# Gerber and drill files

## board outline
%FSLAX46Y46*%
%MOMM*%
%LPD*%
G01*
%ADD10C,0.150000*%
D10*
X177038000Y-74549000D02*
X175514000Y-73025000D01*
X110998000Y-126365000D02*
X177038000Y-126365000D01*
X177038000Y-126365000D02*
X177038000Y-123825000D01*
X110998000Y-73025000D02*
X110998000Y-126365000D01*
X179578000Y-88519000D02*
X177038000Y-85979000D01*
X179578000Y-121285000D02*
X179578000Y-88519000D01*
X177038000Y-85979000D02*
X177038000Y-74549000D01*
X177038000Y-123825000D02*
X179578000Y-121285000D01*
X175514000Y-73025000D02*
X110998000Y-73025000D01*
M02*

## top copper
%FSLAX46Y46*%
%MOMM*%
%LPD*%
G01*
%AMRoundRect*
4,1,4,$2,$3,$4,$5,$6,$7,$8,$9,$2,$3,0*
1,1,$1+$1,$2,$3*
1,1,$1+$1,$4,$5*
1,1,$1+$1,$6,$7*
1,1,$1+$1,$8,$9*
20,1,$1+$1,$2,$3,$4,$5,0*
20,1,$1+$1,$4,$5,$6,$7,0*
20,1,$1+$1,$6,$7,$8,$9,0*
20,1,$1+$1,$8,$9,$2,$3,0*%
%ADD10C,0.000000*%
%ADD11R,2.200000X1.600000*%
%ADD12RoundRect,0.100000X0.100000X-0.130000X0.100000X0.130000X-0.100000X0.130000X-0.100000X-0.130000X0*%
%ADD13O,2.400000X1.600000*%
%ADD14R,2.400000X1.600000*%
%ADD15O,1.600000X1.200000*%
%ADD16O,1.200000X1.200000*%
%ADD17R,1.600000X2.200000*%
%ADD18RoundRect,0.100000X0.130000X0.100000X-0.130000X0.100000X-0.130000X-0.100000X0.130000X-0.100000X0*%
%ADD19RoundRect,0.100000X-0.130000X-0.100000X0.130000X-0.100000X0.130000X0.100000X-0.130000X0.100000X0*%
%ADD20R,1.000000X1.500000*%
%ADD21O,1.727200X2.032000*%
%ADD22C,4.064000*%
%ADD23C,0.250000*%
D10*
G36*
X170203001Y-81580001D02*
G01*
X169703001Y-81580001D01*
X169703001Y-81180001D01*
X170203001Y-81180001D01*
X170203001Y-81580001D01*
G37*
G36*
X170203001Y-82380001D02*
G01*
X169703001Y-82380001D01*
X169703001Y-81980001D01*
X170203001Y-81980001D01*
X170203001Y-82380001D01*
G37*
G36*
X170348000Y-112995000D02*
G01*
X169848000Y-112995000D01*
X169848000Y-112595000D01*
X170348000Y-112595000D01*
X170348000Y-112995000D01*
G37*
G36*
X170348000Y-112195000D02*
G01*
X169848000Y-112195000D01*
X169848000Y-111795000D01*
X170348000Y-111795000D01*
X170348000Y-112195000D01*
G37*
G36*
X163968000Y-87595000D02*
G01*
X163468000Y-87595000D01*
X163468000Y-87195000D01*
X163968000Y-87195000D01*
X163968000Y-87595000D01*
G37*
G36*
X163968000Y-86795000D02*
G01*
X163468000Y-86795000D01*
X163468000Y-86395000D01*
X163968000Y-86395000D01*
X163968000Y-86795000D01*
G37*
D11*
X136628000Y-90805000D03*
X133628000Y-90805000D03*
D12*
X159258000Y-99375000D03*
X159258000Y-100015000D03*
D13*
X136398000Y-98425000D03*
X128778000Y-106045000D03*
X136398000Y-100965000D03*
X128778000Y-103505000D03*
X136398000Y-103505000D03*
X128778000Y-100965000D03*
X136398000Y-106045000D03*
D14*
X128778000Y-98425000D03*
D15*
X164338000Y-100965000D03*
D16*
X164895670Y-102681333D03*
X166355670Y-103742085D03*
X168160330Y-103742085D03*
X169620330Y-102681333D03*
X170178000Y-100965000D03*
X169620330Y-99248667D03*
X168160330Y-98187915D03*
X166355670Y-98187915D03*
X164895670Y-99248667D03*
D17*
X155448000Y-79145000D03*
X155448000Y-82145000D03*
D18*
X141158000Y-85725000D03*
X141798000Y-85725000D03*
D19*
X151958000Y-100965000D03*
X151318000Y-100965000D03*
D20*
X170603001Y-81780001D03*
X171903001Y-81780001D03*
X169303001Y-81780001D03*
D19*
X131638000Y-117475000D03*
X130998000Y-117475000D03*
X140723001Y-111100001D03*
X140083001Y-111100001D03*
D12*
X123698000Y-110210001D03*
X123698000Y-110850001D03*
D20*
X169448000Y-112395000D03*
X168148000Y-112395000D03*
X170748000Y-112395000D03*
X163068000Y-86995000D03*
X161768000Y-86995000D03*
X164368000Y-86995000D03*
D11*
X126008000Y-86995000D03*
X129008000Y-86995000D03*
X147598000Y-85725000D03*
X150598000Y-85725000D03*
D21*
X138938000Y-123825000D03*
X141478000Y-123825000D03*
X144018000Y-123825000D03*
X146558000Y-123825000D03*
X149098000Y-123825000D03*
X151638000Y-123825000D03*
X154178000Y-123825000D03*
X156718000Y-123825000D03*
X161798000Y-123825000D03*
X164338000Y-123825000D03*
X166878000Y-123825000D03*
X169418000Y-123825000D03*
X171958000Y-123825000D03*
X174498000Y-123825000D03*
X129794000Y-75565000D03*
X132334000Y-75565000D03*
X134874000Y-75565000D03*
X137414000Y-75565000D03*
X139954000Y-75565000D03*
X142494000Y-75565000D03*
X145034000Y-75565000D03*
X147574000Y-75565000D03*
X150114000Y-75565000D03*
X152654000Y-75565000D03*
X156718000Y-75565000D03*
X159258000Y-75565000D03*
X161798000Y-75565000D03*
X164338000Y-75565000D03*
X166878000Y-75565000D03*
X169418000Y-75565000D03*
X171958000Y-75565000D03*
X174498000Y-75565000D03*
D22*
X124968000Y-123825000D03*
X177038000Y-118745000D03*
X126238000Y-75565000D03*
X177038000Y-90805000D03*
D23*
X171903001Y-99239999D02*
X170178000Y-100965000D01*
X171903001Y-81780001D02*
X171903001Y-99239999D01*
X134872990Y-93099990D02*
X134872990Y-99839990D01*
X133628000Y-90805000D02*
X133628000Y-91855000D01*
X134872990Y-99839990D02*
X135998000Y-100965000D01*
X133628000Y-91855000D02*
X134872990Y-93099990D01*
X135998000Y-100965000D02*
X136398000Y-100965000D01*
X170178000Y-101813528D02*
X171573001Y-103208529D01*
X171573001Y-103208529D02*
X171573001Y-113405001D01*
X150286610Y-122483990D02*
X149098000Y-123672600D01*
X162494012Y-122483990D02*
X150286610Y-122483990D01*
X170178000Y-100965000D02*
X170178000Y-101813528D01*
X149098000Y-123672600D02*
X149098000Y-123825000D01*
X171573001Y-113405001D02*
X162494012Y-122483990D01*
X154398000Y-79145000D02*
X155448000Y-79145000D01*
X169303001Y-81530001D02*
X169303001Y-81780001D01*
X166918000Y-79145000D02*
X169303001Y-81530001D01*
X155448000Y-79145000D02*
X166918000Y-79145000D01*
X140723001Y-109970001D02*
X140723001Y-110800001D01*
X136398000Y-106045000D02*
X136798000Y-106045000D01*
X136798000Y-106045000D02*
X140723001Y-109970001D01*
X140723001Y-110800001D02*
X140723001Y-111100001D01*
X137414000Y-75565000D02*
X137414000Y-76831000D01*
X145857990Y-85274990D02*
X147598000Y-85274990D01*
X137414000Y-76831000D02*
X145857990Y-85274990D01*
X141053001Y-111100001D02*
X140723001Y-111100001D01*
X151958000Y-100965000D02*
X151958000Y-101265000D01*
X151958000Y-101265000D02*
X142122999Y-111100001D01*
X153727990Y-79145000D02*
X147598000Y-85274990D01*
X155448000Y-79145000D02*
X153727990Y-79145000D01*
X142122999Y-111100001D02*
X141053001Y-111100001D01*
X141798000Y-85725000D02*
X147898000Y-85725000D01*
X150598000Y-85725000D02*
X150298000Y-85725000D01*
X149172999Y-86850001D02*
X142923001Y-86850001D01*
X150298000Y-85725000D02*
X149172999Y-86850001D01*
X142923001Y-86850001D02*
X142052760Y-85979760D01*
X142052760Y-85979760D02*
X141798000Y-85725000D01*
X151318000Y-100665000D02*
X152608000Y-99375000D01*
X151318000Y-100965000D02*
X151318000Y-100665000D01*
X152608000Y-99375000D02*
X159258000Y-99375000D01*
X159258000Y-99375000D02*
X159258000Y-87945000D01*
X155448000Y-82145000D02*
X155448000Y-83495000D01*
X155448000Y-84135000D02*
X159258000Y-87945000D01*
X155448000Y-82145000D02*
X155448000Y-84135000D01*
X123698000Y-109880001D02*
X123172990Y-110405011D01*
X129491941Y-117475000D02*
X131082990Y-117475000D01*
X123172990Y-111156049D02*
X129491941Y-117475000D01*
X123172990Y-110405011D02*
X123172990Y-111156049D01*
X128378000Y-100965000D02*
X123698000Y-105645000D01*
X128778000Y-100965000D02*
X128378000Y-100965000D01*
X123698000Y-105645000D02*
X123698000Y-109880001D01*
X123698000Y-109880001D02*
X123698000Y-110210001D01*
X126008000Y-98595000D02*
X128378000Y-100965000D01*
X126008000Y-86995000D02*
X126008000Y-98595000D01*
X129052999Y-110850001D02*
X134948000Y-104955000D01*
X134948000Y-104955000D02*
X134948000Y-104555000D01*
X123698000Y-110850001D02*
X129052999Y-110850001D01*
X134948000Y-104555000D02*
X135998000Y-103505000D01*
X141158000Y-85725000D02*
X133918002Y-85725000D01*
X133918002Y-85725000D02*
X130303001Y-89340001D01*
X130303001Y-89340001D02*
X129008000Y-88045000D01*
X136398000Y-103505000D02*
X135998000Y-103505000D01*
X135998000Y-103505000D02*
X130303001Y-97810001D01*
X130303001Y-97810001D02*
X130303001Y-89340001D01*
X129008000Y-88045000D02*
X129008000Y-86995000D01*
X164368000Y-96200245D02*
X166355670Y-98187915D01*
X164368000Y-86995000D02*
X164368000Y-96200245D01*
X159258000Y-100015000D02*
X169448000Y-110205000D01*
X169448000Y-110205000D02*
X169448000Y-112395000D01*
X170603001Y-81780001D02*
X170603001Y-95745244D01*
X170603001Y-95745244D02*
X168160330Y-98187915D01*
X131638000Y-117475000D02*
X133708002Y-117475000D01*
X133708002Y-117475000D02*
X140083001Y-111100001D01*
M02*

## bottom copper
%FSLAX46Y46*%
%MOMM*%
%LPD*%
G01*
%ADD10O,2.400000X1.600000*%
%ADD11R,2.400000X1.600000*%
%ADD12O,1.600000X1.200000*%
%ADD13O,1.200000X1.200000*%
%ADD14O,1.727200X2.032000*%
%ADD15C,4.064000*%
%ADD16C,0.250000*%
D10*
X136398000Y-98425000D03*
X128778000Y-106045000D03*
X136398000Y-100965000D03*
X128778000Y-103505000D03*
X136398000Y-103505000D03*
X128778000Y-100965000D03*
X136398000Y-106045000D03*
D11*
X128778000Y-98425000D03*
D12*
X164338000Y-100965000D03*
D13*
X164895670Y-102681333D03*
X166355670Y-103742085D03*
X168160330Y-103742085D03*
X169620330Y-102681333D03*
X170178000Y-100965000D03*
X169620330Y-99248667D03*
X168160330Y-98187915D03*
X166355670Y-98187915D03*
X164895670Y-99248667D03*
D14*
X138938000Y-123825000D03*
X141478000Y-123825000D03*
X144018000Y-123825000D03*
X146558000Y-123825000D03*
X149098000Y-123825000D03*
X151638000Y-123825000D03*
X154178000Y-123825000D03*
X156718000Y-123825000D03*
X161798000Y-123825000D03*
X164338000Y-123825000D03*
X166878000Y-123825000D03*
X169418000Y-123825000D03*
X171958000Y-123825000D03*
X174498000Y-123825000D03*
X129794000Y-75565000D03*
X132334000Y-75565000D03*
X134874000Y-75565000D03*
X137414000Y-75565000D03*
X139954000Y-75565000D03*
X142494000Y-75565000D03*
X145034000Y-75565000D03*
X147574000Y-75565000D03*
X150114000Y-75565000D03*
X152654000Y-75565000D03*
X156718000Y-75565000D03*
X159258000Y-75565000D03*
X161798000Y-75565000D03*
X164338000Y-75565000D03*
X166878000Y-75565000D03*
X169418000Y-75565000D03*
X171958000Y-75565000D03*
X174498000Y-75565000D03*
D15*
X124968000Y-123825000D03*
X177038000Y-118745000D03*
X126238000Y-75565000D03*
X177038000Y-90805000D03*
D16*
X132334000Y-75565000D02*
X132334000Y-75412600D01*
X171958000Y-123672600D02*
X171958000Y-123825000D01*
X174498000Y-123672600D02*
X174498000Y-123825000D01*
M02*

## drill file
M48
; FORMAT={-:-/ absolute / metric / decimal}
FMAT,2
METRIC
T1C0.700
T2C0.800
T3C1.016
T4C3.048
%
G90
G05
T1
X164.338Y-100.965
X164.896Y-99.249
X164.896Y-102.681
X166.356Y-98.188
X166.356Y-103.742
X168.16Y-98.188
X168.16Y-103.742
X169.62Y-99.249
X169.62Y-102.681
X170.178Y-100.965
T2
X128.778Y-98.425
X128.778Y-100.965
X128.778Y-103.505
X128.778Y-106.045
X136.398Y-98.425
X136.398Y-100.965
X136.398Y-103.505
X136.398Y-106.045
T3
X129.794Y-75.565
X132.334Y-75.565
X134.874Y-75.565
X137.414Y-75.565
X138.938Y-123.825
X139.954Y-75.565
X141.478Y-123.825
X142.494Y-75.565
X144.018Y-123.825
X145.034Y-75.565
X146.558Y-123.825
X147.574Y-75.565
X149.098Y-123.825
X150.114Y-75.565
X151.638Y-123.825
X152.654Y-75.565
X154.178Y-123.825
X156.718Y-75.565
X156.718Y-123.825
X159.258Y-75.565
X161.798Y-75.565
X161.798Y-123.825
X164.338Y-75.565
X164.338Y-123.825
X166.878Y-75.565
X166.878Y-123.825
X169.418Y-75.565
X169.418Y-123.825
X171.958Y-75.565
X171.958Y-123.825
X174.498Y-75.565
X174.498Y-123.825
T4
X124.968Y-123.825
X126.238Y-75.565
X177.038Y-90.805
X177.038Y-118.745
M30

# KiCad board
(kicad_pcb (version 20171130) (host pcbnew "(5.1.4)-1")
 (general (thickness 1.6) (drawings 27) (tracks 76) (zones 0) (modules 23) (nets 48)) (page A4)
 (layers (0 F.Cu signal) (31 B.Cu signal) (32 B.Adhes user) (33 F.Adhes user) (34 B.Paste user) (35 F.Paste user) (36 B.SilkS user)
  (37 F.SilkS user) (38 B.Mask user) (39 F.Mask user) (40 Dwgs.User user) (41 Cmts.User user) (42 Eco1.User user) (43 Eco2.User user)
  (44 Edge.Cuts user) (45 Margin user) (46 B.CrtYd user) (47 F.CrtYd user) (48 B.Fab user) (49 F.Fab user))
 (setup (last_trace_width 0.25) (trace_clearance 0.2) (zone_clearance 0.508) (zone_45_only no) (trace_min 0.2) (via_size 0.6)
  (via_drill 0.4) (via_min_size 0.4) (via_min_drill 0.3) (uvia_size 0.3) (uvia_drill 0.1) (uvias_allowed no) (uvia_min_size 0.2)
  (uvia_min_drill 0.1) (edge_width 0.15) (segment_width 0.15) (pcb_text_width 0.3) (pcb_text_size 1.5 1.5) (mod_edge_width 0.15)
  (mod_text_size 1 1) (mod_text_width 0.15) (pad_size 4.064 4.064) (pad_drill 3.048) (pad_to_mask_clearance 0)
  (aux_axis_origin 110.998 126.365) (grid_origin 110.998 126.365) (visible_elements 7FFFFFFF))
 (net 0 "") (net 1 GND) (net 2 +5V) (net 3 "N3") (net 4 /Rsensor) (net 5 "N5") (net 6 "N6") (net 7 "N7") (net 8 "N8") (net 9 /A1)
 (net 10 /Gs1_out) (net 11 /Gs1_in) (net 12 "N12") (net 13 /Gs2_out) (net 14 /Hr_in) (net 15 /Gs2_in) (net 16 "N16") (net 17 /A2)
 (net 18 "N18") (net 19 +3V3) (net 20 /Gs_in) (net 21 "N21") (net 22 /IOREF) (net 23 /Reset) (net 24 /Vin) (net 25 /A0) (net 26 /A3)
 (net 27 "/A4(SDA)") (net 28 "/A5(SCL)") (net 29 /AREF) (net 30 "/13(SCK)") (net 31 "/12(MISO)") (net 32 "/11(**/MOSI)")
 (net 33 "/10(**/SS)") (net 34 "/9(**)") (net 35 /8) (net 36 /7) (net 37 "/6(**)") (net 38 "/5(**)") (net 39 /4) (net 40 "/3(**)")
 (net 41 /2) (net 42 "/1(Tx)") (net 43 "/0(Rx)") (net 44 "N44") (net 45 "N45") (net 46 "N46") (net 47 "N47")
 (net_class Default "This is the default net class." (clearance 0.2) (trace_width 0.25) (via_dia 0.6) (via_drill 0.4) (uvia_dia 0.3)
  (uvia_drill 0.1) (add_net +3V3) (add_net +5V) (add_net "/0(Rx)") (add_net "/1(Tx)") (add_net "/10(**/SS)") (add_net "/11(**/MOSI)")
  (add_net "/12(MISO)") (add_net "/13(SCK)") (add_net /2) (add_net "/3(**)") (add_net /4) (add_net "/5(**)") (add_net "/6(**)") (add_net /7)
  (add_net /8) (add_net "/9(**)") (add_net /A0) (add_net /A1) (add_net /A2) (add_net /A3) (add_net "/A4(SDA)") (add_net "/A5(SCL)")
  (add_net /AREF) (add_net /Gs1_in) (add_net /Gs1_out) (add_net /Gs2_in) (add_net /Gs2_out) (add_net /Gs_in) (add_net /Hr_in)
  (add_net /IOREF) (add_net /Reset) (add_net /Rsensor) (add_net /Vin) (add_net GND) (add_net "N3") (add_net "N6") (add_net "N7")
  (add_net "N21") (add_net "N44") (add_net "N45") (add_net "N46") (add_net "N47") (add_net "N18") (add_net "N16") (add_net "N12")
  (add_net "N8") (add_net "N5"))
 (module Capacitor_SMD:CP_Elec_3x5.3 (layer F.Cu) (at 135.128 90.805)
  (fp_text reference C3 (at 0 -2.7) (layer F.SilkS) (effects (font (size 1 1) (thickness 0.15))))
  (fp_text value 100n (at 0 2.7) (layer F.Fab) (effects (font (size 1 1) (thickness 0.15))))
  (pad 2 smd rect (at 1.5 0) (size 2.2 1.6) (layers F.Cu F.Paste F.Mask) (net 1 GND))
  (pad 1 smd rect (at -1.5 0) (size 2.2 1.6) (layers F.Cu F.Paste F.Mask) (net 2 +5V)))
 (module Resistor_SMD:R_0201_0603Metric (layer F.Cu) (at 159.258 99.695 90)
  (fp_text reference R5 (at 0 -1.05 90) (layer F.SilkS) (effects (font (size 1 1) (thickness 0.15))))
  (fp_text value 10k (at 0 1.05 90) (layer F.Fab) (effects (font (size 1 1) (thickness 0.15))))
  (pad 2 smd roundrect (at 0.32 0 90) (size 0.46 0.4) (layers F.Cu F.Mask) (roundrect_rratio 0.25) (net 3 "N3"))
  (pad 1 smd roundrect (at -0.32 0 90) (size 0.46 0.4) (layers F.Cu F.Mask) (roundrect_rratio 0.25) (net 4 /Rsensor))
  (pad "" smd roundrect (at 0.345 0 90) (size 0.318 0.36) (layers F.Paste) (roundrect_rratio 0.25))
  (pad "" smd roundrect (at -0.345 0 90) (size 0.318 0.36) (layers F.Paste) (roundrect_rratio 0.25)))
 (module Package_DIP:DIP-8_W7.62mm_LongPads (layer F.Cu) (at 128.778 98.425)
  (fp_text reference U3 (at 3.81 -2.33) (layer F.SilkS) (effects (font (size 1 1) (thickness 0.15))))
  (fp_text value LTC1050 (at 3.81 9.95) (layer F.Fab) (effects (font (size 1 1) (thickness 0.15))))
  (pad 8 thru_hole oval (at 7.62 0) (size 2.4 1.6) (drill 0.8) (layers *.Cu *.Mask) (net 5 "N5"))
  (pad 4 thru_hole oval (at 0 7.62) (size 2.4 1.6) (drill 0.8) (layers *.Cu *.Mask) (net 1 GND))
  (pad 7 thru_hole oval (at 7.62 2.54) (size 2.4 1.6) (drill 0.8) (layers *.Cu *.Mask) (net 2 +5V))
  (pad 3 thru_hole oval (at 0 5.08) (size 2.4 1.6) (drill 0.8) (layers *.Cu *.Mask) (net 3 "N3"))
  (pad 6 thru_hole oval (at 7.62 5.08) (size 2.4 1.6) (drill 0.8) (layers *.Cu *.Mask) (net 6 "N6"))
  (pad 2 thru_hole oval (at 0 2.54) (size 2.4 1.6) (drill 0.8) (layers *.Cu *.Mask) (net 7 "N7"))
  (pad 5 thru_hole oval (at 7.62 7.62) (size 2.4 1.6) (drill 0.8) (layers *.Cu *.Mask) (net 1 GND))
  (pad 1 thru_hole rect (at 0 0) (size 2.4 1.6) (drill 0.8) (layers *.Cu *.Mask) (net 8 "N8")))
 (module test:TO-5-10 (layer F.Cu) (at 164.338 100.965)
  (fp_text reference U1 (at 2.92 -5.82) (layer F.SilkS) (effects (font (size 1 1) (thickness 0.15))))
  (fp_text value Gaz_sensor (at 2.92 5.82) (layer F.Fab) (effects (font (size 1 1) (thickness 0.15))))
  (pad 1 thru_hole oval (at 0 0) (size 1.6 1.2) (drill 0.7) (layers *.Cu *.Mask) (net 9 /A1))
  (pad 2 thru_hole oval (at 0.55767 1.716333) (size 1.2 1.2) (drill 0.7) (layers *.Cu *.Mask) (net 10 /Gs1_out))
  (pad 3 thru_hole oval (at 2.01767 2.777085) (size 1.2 1.2) (drill 0.7) (layers *.Cu *.Mask) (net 1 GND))
  (pad 4 thru_hole oval (at 3.82233 2.777085) (size 1.2 1.2) (drill 0.7) (layers *.Cu *.Mask) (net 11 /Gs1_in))
  (pad 5 thru_hole oval (at 5.28233 1.716333) (size 1.2 1.2) (drill 0.7) (layers *.Cu *.Mask) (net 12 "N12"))
  (pad 6 thru_hole oval (at 5.84 0) (size 1.2 1.2) (drill 0.7) (layers *.Cu *.Mask) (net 2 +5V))
  (pad 7 thru_hole oval (at 5.28233 -1.716333) (size 1.2 1.2) (drill 0.7) (layers *.Cu *.Mask) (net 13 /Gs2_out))
  (pad 8 thru_hole oval (at 3.82233 -2.777085) (size 1.2 1.2) (drill 0.7) (layers *.Cu *.Mask) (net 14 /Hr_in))
  (pad 9 thru_hole oval (at 2.01767 -2.777085) (size 1.2 1.2) (drill 0.7) (layers *.Cu *.Mask) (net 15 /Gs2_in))
  (pad 10 thru_hole oval (at 0.55767 -1.716333) (size 1.2 1.2) (drill 0.7) (layers *.Cu *.Mask) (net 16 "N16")))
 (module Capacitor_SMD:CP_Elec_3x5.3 (layer F.Cu) (at 155.448 80.645 90)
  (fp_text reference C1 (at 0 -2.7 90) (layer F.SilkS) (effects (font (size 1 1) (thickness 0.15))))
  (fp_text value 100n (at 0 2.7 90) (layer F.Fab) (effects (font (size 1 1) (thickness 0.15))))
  (pad 2 smd rect (at 1.5 0 90) (size 2.2 1.6) (layers F.Cu F.Paste F.Mask) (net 1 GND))
  (pad 1 smd rect (at -1.5 0 90) (size 2.2 1.6) (layers F.Cu F.Paste F.Mask) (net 3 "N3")))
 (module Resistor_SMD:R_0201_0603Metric (layer F.Cu) (at 141.478 85.725 180)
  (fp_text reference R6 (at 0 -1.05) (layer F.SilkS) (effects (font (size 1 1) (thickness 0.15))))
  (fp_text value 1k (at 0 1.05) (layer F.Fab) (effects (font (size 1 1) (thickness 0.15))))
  (pad 2 smd roundrect (at 0.32 0 180) (size 0.46 0.4) (layers F.Cu F.Mask) (roundrect_rratio 0.25) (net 6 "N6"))
  (pad 1 smd roundrect (at -0.32 0 180) (size 0.46 0.4) (layers F.Cu F.Mask) (roundrect_rratio 0.25) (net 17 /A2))
  (pad "" smd roundrect (at 0.345 0 180) (size 0.318 0.36) (layers F.Paste) (roundrect_rratio 0.25))
  (pad "" smd roundrect (at -0.345 0 180) (size 0.318 0.36) (layers F.Paste) (roundrect_rratio 0.25)))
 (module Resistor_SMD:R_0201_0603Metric (layer F.Cu) (at 151.638 100.965)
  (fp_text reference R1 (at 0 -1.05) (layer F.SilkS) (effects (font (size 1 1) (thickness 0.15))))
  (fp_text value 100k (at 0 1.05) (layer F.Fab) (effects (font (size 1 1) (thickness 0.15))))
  (pad 2 smd roundrect (at 0.32 0) (size 0.46 0.4) (layers F.Cu F.Mask) (roundrect_rratio 0.25) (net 1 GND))
  (pad 1 smd roundrect (at -0.32 0) (size 0.46 0.4) (layers F.Cu F.Mask) (roundrect_rratio 0.25) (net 3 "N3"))
  (pad "" smd roundrect (at 0.345 0) (size 0.318 0.36) (layers F.Paste) (roundrect_rratio 0.25))
  (pad "" smd roundrect (at -0.345 0) (size 0.318 0.36) (layers F.Paste) (roundrect_rratio 0.25)))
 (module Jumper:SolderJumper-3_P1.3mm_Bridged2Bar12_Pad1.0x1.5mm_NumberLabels (layer F.Cu) (at 170.603001 81.780001)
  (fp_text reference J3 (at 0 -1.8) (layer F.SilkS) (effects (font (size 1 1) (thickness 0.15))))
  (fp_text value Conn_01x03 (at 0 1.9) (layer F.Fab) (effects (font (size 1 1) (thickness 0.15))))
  (fp_poly (pts (xy -0.9 -0.6) (xy -0.4 -0.6) (xy -0.4 -0.2) (xy -0.9 -0.2)) (layer F.Cu) (width 0))
  (fp_poly (pts (xy -0.9 0.2) (xy -0.4 0.2) (xy -0.4 0.6) (xy -0.9 0.6)) (layer F.Cu) (width 0))
  (pad 2 smd rect (at 0 0) (size 1 1.5) (layers F.Cu F.Mask) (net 14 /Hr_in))
  (pad 3 smd rect (at 1.3 0) (size 1 1.5) (layers F.Cu F.Mask) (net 2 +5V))
  (pad 1 smd rect (at -1.3 0) (size 1 1.5) (layers F.Cu F.Mask) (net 1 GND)))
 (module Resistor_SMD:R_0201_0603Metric (layer F.Cu) (at 131.318 117.475)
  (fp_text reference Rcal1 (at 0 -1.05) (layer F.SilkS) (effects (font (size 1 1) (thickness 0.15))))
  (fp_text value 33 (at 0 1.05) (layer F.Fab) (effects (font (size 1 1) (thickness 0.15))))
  (pad 2 smd roundrect (at 0.32 0) (size 0.46 0.4) (layers F.Cu F.Mask) (roundrect_rratio 0.25) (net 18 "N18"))
  (pad 1 smd roundrect (at -0.32 0) (size 0.46 0.4) (layers F.Cu F.Mask) (roundrect_rratio 0.25) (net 7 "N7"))
  (pad "" smd roundrect (at 0.345 0) (size 0.318 0.36) (layers F.Paste) (roundrect_rratio 0.25))
  (pad "" smd roundrect (at -0.345 0) (size 0.318 0.36) (layers F.Paste) (roundrect_rratio 0.25)))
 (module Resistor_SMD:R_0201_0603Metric (layer F.Cu) (at 140.403001 111.100001)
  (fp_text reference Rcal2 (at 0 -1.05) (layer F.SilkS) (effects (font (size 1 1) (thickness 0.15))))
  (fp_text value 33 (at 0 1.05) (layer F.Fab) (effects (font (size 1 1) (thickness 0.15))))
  (pad 2 smd roundrect (at 0.32 0) (size 0.46 0.4) (layers F.Cu F.Mask) (roundrect_rratio 0.25) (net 1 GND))
  (pad 1 smd roundrect (at -0.32 0) (size 0.46 0.4) (layers F.Cu F.Mask) (roundrect_rratio 0.25) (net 18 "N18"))
  (pad "" smd roundrect (at 0.345 0) (size 0.318 0.36) (layers F.Paste) (roundrect_rratio 0.25))
  (pad "" smd roundrect (at -0.345 0) (size 0.318 0.36) (layers F.Paste) (roundrect_rratio 0.25)))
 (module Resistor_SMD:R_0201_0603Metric (layer F.Cu) (at 123.698 110.530001 90)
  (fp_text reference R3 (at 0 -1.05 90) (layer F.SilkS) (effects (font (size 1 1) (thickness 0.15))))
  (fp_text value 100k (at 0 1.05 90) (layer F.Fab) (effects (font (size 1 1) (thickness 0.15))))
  (pad 2 smd roundrect (at 0.32 0 90) (size 0.46 0.4) (layers F.Cu F.Mask) (roundrect_rratio 0.25) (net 7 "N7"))
  (pad 1 smd roundrect (at -0.32 0 90) (size 0.46 0.4) (layers F.Cu F.Mask) (roundrect_rratio 0.25) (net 6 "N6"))
  (pad "" smd roundrect (at 0.345 0 90) (size 0.318 0.36) (layers F.Paste) (roundrect_rratio 0.25))
  (pad "" smd roundrect (at -0.345 0 90) (size 0.318 0.36) (layers F.Paste) (roundrect_rratio 0.25)))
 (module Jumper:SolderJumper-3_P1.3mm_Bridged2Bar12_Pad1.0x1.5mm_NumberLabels (layer F.Cu) (at 169.448 112.395 180)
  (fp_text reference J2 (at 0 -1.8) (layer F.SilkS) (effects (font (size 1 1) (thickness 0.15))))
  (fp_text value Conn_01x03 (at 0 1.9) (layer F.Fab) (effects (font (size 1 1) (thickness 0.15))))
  (fp_poly (pts (xy -0.9 -0.6) (xy -0.4 -0.6) (xy -0.4 -0.2) (xy -0.9 -0.2)) (layer F.Cu) (width 0))
  (fp_poly (pts (xy -0.9 0.2) (xy -0.4 0.2) (xy -0.4 0.6) (xy -0.9 0.6)) (layer F.Cu) (width 0))
  (pad 2 smd rect (at 0 0 180) (size 1 1.5) (layers F.Cu F.Mask) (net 4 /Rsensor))
  (pad 3 smd rect (at 1.3 0 180) (size 1 1.5) (layers F.Cu F.Mask) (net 10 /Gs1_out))
  (pad 1 smd rect (at -1.3 0 180) (size 1 1.5) (layers F.Cu F.Mask) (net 13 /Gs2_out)))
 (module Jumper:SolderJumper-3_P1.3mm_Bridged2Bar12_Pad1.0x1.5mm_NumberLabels (layer F.Cu) (at 163.068 86.995 180)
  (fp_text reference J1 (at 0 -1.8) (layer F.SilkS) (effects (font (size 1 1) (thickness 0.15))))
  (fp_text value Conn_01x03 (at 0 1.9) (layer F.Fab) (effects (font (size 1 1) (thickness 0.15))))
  (fp_poly (pts (xy -0.9 -0.6) (xy -0.4 -0.6) (xy -0.4 -0.2) (xy -0.9 -0.2)) (layer F.Cu) (width 0))
  (fp_poly (pts (xy -0.9 0.2) (xy -0.4 0.2) (xy -0.4 0.6) (xy -0.9 0.6)) (layer F.Cu) (width 0))
  (pad 2 smd rect (at 0 0 180) (size 1 1.5) (layers F.Cu F.Mask) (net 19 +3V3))
  (pad 3 smd rect (at 1.3 0 180) (size 1 1.5) (layers F.Cu F.Mask) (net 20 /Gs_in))
  (pad 1 smd rect (at -1.3 0 180) (size 1 1.5) (layers F.Cu F.Mask) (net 15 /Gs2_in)))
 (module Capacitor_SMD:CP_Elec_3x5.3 (layer F.Cu) (at 127.508 86.995 180)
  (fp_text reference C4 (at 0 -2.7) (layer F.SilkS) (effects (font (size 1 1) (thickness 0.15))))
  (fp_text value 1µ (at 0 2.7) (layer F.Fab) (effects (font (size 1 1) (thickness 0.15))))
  (pad 2 smd rect (at 1.5 0 180) (size 2.2 1.6) (layers F.Cu F.Paste F.Mask) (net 7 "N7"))
  (pad 1 smd rect (at -1.5 0 180) (size 2.2 1.6) (layers F.Cu F.Paste F.Mask) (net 6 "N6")))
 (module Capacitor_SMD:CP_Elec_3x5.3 (layer F.Cu) (at 149.098 85.725 180)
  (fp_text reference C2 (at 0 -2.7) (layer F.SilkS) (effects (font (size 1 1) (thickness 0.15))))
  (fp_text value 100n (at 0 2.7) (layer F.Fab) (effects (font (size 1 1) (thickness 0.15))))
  (pad 2 smd rect (at 1.5 0 180) (size 2.2 1.6) (layers F.Cu F.Paste F.Mask) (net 1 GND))
  (pad 1 smd rect (at -1.5 0 180) (size 2.2 1.6) (layers F.Cu F.Paste F.Mask) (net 17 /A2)))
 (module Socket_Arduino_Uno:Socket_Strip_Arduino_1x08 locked (layer F.Cu) (at 138.938 123.825)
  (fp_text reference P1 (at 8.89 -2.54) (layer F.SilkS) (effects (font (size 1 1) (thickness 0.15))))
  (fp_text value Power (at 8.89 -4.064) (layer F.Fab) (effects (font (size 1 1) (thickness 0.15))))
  (pad 1 thru_hole oval (at 0 0) (size 1.7272 2.032) (drill 1.016) (layers *.Cu *.Mask F.SilkS) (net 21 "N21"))
  (pad 2 thru_hole oval (at 2.54 0) (size 1.7272 2.032) (drill 1.016) (layers *.Cu *.Mask F.SilkS) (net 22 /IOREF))
  (pad 3 thru_hole oval (at 5.08 0) (size 1.7272 2.032) (drill 1.016) (layers *.Cu *.Mask F.SilkS) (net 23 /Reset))
  (pad 4 thru_hole oval (at 7.62 0) (size 1.7272 2.032) (drill 1.016) (layers *.Cu *.Mask F.SilkS) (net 19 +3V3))
  (pad 5 thru_hole oval (at 10.16 0) (size 1.7272 2.032) (drill 1.016) (layers *.Cu *.Mask F.SilkS) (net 2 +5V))
  (pad 6 thru_hole oval (at 12.7 0) (size 1.7272 2.032) (drill 1.016) (layers *.Cu *.Mask F.SilkS) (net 1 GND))
  (pad 7 thru_hole oval (at 15.24 0) (size 1.7272 2.032) (drill 1.016) (layers *.Cu *.Mask F.SilkS) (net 1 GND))
  (pad 8 thru_hole oval (at 17.78 0) (size 1.7272 2.032) (drill 1.016) (layers *.Cu *.Mask F.SilkS) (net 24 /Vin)))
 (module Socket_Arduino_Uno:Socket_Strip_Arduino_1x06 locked (layer F.Cu) (at 161.798 123.825)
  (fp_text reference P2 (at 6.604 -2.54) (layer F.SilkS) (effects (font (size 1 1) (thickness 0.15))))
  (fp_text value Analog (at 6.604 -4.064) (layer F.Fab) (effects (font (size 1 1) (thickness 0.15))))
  (pad 1 thru_hole oval (at 0 0) (size 1.7272 2.032) (drill 1.016) (layers *.Cu *.Mask F.SilkS) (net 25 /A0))
  (pad 2 thru_hole oval (at 2.54 0) (size 1.7272 2.032) (drill 1.016) (layers *.Cu *.Mask F.SilkS) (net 9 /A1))
  (pad 3 thru_hole oval (at 5.08 0) (size 1.7272 2.032) (drill 1.016) (layers *.Cu *.Mask F.SilkS) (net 17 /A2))
  (pad 4 thru_hole oval (at 7.62 0) (size 1.7272 2.032) (drill 1.016) (layers *.Cu *.Mask F.SilkS) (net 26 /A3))
  (pad 5 thru_hole oval (at 10.16 0) (size 1.7272 2.032) (drill 1.016) (layers *.Cu *.Mask F.SilkS) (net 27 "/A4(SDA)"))
  (pad 6 thru_hole oval (at 12.7 0) (size 1.7272 2.032) (drill 1.016) (layers *.Cu *.Mask F.SilkS) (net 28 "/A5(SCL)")))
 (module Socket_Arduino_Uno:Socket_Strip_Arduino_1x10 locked (layer F.Cu) (at 129.794 75.565)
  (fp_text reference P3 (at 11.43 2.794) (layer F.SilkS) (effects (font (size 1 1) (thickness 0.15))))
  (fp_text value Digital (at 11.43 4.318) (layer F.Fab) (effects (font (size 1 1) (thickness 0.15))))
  (pad 1 thru_hole oval (at 0 0) (size 1.7272 2.032) (drill 1.016) (layers *.Cu *.Mask F.SilkS) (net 28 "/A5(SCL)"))
  (pad 2 thru_hole oval (at 2.54 0) (size 1.7272 2.032) (drill 1.016) (layers *.Cu *.Mask F.SilkS) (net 27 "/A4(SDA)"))
  (pad 3 thru_hole oval (at 5.08 0) (size 1.7272 2.032) (drill 1.016) (layers *.Cu *.Mask F.SilkS) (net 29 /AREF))
  (pad 4 thru_hole oval (at 7.62 0) (size 1.7272 2.032) (drill 1.016) (layers *.Cu *.Mask F.SilkS) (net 1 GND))
  (pad 5 thru_hole oval (at 10.16 0) (size 1.7272 2.032) (drill 1.016) (layers *.Cu *.Mask F.SilkS) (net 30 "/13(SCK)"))
  (pad 6 thru_hole oval (at 12.7 0) (size 1.7272 2.032) (drill 1.016) (layers *.Cu *.Mask F.SilkS) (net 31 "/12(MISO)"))
  (pad 7 thru_hole oval (at 15.24 0) (size 1.7272 2.032) (drill 1.016) (layers *.Cu *.Mask F.SilkS) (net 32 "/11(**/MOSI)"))
  (pad 8 thru_hole oval (at 17.78 0) (size 1.7272 2.032) (drill 1.016) (layers *.Cu *.Mask F.SilkS) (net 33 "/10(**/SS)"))
  (pad 9 thru_hole oval (at 20.32 0) (size 1.7272 2.032) (drill 1.016) (layers *.Cu *.Mask F.SilkS) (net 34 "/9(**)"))
  (pad 10 thru_hole oval (at 22.86 0) (size 1.7272 2.032) (drill 1.016) (layers *.Cu *.Mask F.SilkS) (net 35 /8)))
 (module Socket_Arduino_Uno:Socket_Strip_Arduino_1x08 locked (layer F.Cu) (at 156.718 75.565)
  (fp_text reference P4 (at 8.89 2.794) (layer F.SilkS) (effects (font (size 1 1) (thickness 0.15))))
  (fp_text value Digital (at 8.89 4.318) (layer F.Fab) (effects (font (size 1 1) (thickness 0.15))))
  (pad 1 thru_hole oval (at 0 0) (size 1.7272 2.032) (drill 1.016) (layers *.Cu *.Mask F.SilkS) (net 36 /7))
  (pad 2 thru_hole oval (at 2.54 0) (size 1.7272 2.032) (drill 1.016) (layers *.Cu *.Mask F.SilkS) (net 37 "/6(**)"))
  (pad 3 thru_hole oval (at 5.08 0) (size 1.7272 2.032) (drill 1.016) (layers *.Cu *.Mask F.SilkS) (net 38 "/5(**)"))
  (pad 4 thru_hole oval (at 7.62 0) (size 1.7272 2.032) (drill 1.016) (layers *.Cu *.Mask F.SilkS) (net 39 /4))
  (pad 5 thru_hole oval (at 10.16 0) (size 1.7272 2.032) (drill 1.016) (layers *.Cu *.Mask F.SilkS) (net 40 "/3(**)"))
  (pad 6 thru_hole oval (at 12.7 0) (size 1.7272 2.032) (drill 1.016) (layers *.Cu *.Mask F.SilkS) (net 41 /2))
  (pad 7 thru_hole oval (at 15.24 0) (size 1.7272 2.032) (drill 1.016) (layers *.Cu *.Mask F.SilkS) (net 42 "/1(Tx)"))
  (pad 8 thru_hole oval (at 17.78 0) (size 1.7272 2.032) (drill 1.016) (layers *.Cu *.Mask F.SilkS) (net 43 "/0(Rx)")))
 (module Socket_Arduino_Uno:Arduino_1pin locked (layer F.Cu) (at 124.968 123.825)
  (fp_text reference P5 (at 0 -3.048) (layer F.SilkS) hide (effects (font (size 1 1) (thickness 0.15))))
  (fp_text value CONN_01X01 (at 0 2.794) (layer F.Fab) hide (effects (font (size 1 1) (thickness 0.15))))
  (pad 1 thru_hole circle (at 0 0) (size 4.064 4.064) (drill 3.048) (layers *.Cu *.Mask F.SilkS) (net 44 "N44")))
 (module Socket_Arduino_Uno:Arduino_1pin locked (layer F.Cu) (at 177.038 118.745)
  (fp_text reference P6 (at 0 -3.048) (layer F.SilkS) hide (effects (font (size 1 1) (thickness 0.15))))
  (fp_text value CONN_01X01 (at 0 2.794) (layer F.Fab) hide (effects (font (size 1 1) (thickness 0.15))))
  (pad 1 thru_hole circle (at 0 0) (size 4.064 4.064) (drill 3.048) (layers *.Cu *.Mask F.SilkS) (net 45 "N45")))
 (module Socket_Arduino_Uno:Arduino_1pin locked (layer F.Cu) (at 126.238 75.565)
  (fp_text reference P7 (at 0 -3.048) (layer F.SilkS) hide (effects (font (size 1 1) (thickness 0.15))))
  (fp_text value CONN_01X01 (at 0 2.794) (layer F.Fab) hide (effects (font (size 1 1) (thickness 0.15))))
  (pad 1 thru_hole circle (at 0 0) (size 4.064 4.064) (drill 3.048) (layers *.Cu *.Mask F.SilkS) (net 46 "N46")))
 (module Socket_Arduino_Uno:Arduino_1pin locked (layer F.Cu) (at 177.038 90.805)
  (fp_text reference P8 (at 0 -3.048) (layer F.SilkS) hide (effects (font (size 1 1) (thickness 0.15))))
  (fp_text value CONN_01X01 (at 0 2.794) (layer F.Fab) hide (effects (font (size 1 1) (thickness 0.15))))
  (pad 1 thru_hole circle (at 0 0) (size 4.064 4.064) (drill 3.048) (layers *.Cu *.Mask F.SilkS) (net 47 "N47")))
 (gr_line (start 177.038 74.549) (end 175.514 73.025) (angle 90) (layer Edge.Cuts) (width 0.15))
 (gr_line (start 110.998 126.365) (end 177.038 126.365) (angle 90) (layer Edge.Cuts) (width 0.15))
 (gr_line (start 177.038 126.365) (end 177.038 123.825) (angle 90) (layer Edge.Cuts) (width 0.15))
 (gr_line (start 110.998 73.025) (end 110.998 126.365) (angle 90) (layer Edge.Cuts) (width 0.15))
 (gr_line (start 179.578 88.519) (end 177.038 85.979) (angle 90) (layer Edge.Cuts) (width 0.15))
 (gr_line (start 179.578 121.285) (end 179.578 88.519) (angle 90) (layer Edge.Cuts) (width 0.15))
 (gr_line (start 177.038 85.979) (end 177.038 74.549) (angle 90) (layer Edge.Cuts) (width 0.15))
 (gr_line (start 177.038 123.825) (end 179.578 121.285) (angle 90) (layer Edge.Cuts) (width 0.15))
 (gr_line (start 175.514 73.025) (end 110.998 73.025) (angle 90) (layer Edge.Cuts) (width 0.15))
 (segment (start 171.903001 99.239999) (end 170.178 100.965) (width 0.25) (layer F.Cu) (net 2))
 (segment (start 171.903001 81.780001) (end 171.903001 99.239999) (width 0.25) (layer F.Cu) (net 2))
 (segment (start 134.87299 93.09999) (end 134.87299 99.83999) (width 0.25) (layer F.Cu) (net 2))
 (segment (start 133.628 90.805) (end 133.628 91.855) (width 0.25) (layer F.Cu) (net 2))
 (segment (start 134.87299 99.83999) (end 135.998 100.965) (width 0.25) (layer F.Cu) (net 2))
 (segment (start 133.628 91.855) (end 134.87299 93.09999) (width 0.25) (layer F.Cu) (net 2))
 (segment (start 135.998 100.965) (end 136.398 100.965) (width 0.25) (layer F.Cu) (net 2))
 (segment (start 170.178 101.813528) (end 171.573001 103.208529) (width 0.25) (layer F.Cu) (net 2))
 (segment (start 171.573001 103.208529) (end 171.573001 113.405001) (width 0.25) (layer F.Cu) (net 2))
 (segment (start 150.28661 122.48399) (end 149.098 123.6726) (width 0.25) (layer F.Cu) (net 2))
 (segment (start 162.494012 122.48399) (end 150.28661 122.48399) (width 0.25) (layer F.Cu) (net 2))
 (segment (start 170.178 100.965) (end 170.178 101.813528) (width 0.25) (layer F.Cu) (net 2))
 (segment (start 149.098 123.6726) (end 149.098 123.825) (width 0.25) (layer F.Cu) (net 2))
 (segment (start 171.573001 113.405001) (end 162.494012 122.48399) (width 0.25) (layer F.Cu) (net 2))
 (segment (start 154.398 79.145) (end 155.448 79.145) (width 0.25) (layer F.Cu) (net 1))
 (segment (start 169.303001 81.530001) (end 169.303001 81.780001) (width 0.25) (layer F.Cu) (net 1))
 (segment (start 166.918 79.145) (end 169.303001 81.530001) (width 0.25) (layer F.Cu) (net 1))
 (segment (start 155.448 79.145) (end 166.918 79.145) (width 0.25) (layer F.Cu) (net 1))
 (segment (start 140.723001 109.970001) (end 140.723001 110.800001) (width 0.25) (layer F.Cu) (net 1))
 (segment (start 136.398 106.045) (end 136.798 106.045) (width 0.25) (layer F.Cu) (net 1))
 (segment (start 136.798 106.045) (end 140.723001 109.970001) (width 0.25) (layer F.Cu) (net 1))
 (segment (start 140.723001 110.800001) (end 140.723001 111.100001) (width 0.25) (layer F.Cu) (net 1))
 (segment (start 137.414 75.565) (end 137.414 76.831) (width 0.25) (layer F.Cu) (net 1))
 (segment (start 145.85799 85.27499) (end 147.598 85.27499) (width 0.25) (layer F.Cu) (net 1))
 (segment (start 137.414 76.831) (end 145.85799 85.27499) (width 0.25) (layer F.Cu) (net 1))
 (segment (start 141.053001 111.100001) (end 140.723001 111.100001) (width 0.25) (layer F.Cu) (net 1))
 (segment (start 151.958 100.965) (end 151.958 101.265) (width 0.25) (layer F.Cu) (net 1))
 (segment (start 151.958 101.265) (end 142.122999 111.100001) (width 0.25) (layer F.Cu) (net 1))
 (segment (start 153.72799 79.145) (end 147.598 85.27499) (width 0.25) (layer F.Cu) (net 1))
 (segment (start 155.448 79.145) (end 153.72799 79.145) (width 0.25) (layer F.Cu) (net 1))
 (segment (start 142.122999 111.100001) (end 141.053001 111.100001) (width 0.25) (layer F.Cu) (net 1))
 (segment (start 141.798 85.725) (end 147.898 85.725) (width 0.25) (layer F.Cu) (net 17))
 (segment (start 150.598 85.725) (end 150.298 85.725) (width 0.25) (layer F.Cu) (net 17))
 (segment (start 149.172999 86.850001) (end 142.923001 86.850001) (width 0.25) (layer F.Cu) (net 17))
 (segment (start 150.298 85.725) (end 149.172999 86.850001) (width 0.25) (layer F.Cu) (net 17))
 (segment (start 142.923001 86.850001) (end 142.05276 85.97976) (width 0.25) (layer F.Cu) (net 17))
 (segment (start 142.05276 85.97976) (end 141.798 85.725) (width 0.25) (layer F.Cu) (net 17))
 (segment (start 132.334 75.565) (end 132.334 75.4126) (width 0.25) (layer B.Cu) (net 27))
 (segment (start 171.958 123.6726) (end 171.958 123.825) (width 0.25) (layer B.Cu) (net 27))
 (segment (start 174.498 123.6726) (end 174.498 123.825) (width 0.25) (layer B.Cu) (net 28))
 (segment (start 151.318 100.665) (end 152.608 99.375) (width 0.25) (layer F.Cu) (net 3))
 (segment (start 151.318 100.965) (end 151.318 100.665) (width 0.25) (layer F.Cu) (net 3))
 (segment (start 152.608 99.375) (end 159.258 99.375) (width 0.25) (layer F.Cu) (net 3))
 (segment (start 159.258 99.375) (end 159.258 87.945) (width 0.25) (layer F.Cu) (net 3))
 (segment (start 155.448 82.145) (end 155.448 83.495) (width 0.25) (layer F.Cu) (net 3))
 (segment (start 155.448 84.135) (end 159.258 87.945) (width 0.25) (layer F.Cu) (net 3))
 (segment (start 155.448 82.145) (end 155.448 84.135) (width 0.25) (layer F.Cu) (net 3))
 (segment (start 123.698 109.880001) (end 123.17299 110.405011) (width 0.25) (layer F.Cu) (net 7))
 (segment (start 129.491941 117.475) (end 131.08299 117.475) (width 0.25) (layer F.Cu) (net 7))
 (segment (start 123.17299 111.156049) (end 129.491941 117.475) (width 0.25) (layer F.Cu) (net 7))
 (segment (start 123.17299 110.405011) (end 123.17299 111.156049) (width 0.25) (layer F.Cu) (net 7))
 (segment (start 128.378 100.965) (end 123.698 105.645) (width 0.25) (layer F.Cu) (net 7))
 (segment (start 128.778 100.965) (end 128.378 100.965) (width 0.25) (layer F.Cu) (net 7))
 (segment (start 123.698 105.645) (end 123.698 109.880001) (width 0.25) (layer F.Cu) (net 7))
 (segment (start 123.698 109.880001) (end 123.698 110.210001) (width 0.25) (layer F.Cu) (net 7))
 (segment (start 126.008 98.595) (end 128.378 100.965) (width 0.25) (layer F.Cu) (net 7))
 (segment (start 126.008 86.995) (end 126.008 98.595) (width 0.25) (layer F.Cu) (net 7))
 (segment (start 129.052999 110.850001) (end 134.948 104.955) (width 0.25) (layer F.Cu) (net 6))
 (segment (start 134.948 104.955) (end 134.948 104.555) (width 0.25) (layer F.Cu) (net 6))
 (segment (start 123.698 110.850001) (end 129.052999 110.850001) (width 0.25) (layer F.Cu) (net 6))
 (segment (start 134.948 104.555) (end 135.998 103.505) (width 0.25) (layer F.Cu) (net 6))
 (segment (start 141.158 85.725) (end 133.918002 85.725) (width 0.25) (layer F.Cu) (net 6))
 (segment (start 133.918002 85.725) (end 130.303001 89.340001) (width 0.25) (layer F.Cu) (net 6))
 (segment (start 130.303001 89.340001) (end 129.008 88.045) (width 0.25) (layer F.Cu) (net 6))
 (segment (start 136.398 103.505) (end 135.998 103.505) (width 0.25) (layer F.Cu) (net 6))
 (segment (start 135.998 103.505) (end 130.303001 97.810001) (width 0.25) (layer F.Cu) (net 6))
 (segment (start 130.303001 97.810001) (end 130.303001 89.340001) (width 0.25) (layer F.Cu) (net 6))
 (segment (start 129.008 88.045) (end 129.008 86.995) (width 0.25) (layer F.Cu) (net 6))
 (segment (start 164.368 96.200245) (end 166.35567 98.187915) (width 0.25) (layer F.Cu) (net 15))
 (segment (start 164.368 86.995) (end 164.368 96.200245) (width 0.25) (layer F.Cu) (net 15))
 (segment (start 159.258 100.015) (end 169.448 110.205) (width 0.25) (layer F.Cu) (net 4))
 (segment (start 169.448 110.205) (end 169.448 112.395) (width 0.25) (layer F.Cu) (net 4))
 (segment (start 170.603001 81.780001) (end 170.603001 95.745244) (width 0.25) (layer F.Cu) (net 14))
 (segment (start 170.603001 95.745244) (end 168.16033 98.187915) (width 0.25) (layer F.Cu) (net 14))
 (segment (start 131.638 117.475) (end 133.708002 117.475) (width 0.25) (layer F.Cu) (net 18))
 (segment (start 133.708002 117.475) (end 140.083001 111.100001) (width 0.25) (layer F.Cu) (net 18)))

